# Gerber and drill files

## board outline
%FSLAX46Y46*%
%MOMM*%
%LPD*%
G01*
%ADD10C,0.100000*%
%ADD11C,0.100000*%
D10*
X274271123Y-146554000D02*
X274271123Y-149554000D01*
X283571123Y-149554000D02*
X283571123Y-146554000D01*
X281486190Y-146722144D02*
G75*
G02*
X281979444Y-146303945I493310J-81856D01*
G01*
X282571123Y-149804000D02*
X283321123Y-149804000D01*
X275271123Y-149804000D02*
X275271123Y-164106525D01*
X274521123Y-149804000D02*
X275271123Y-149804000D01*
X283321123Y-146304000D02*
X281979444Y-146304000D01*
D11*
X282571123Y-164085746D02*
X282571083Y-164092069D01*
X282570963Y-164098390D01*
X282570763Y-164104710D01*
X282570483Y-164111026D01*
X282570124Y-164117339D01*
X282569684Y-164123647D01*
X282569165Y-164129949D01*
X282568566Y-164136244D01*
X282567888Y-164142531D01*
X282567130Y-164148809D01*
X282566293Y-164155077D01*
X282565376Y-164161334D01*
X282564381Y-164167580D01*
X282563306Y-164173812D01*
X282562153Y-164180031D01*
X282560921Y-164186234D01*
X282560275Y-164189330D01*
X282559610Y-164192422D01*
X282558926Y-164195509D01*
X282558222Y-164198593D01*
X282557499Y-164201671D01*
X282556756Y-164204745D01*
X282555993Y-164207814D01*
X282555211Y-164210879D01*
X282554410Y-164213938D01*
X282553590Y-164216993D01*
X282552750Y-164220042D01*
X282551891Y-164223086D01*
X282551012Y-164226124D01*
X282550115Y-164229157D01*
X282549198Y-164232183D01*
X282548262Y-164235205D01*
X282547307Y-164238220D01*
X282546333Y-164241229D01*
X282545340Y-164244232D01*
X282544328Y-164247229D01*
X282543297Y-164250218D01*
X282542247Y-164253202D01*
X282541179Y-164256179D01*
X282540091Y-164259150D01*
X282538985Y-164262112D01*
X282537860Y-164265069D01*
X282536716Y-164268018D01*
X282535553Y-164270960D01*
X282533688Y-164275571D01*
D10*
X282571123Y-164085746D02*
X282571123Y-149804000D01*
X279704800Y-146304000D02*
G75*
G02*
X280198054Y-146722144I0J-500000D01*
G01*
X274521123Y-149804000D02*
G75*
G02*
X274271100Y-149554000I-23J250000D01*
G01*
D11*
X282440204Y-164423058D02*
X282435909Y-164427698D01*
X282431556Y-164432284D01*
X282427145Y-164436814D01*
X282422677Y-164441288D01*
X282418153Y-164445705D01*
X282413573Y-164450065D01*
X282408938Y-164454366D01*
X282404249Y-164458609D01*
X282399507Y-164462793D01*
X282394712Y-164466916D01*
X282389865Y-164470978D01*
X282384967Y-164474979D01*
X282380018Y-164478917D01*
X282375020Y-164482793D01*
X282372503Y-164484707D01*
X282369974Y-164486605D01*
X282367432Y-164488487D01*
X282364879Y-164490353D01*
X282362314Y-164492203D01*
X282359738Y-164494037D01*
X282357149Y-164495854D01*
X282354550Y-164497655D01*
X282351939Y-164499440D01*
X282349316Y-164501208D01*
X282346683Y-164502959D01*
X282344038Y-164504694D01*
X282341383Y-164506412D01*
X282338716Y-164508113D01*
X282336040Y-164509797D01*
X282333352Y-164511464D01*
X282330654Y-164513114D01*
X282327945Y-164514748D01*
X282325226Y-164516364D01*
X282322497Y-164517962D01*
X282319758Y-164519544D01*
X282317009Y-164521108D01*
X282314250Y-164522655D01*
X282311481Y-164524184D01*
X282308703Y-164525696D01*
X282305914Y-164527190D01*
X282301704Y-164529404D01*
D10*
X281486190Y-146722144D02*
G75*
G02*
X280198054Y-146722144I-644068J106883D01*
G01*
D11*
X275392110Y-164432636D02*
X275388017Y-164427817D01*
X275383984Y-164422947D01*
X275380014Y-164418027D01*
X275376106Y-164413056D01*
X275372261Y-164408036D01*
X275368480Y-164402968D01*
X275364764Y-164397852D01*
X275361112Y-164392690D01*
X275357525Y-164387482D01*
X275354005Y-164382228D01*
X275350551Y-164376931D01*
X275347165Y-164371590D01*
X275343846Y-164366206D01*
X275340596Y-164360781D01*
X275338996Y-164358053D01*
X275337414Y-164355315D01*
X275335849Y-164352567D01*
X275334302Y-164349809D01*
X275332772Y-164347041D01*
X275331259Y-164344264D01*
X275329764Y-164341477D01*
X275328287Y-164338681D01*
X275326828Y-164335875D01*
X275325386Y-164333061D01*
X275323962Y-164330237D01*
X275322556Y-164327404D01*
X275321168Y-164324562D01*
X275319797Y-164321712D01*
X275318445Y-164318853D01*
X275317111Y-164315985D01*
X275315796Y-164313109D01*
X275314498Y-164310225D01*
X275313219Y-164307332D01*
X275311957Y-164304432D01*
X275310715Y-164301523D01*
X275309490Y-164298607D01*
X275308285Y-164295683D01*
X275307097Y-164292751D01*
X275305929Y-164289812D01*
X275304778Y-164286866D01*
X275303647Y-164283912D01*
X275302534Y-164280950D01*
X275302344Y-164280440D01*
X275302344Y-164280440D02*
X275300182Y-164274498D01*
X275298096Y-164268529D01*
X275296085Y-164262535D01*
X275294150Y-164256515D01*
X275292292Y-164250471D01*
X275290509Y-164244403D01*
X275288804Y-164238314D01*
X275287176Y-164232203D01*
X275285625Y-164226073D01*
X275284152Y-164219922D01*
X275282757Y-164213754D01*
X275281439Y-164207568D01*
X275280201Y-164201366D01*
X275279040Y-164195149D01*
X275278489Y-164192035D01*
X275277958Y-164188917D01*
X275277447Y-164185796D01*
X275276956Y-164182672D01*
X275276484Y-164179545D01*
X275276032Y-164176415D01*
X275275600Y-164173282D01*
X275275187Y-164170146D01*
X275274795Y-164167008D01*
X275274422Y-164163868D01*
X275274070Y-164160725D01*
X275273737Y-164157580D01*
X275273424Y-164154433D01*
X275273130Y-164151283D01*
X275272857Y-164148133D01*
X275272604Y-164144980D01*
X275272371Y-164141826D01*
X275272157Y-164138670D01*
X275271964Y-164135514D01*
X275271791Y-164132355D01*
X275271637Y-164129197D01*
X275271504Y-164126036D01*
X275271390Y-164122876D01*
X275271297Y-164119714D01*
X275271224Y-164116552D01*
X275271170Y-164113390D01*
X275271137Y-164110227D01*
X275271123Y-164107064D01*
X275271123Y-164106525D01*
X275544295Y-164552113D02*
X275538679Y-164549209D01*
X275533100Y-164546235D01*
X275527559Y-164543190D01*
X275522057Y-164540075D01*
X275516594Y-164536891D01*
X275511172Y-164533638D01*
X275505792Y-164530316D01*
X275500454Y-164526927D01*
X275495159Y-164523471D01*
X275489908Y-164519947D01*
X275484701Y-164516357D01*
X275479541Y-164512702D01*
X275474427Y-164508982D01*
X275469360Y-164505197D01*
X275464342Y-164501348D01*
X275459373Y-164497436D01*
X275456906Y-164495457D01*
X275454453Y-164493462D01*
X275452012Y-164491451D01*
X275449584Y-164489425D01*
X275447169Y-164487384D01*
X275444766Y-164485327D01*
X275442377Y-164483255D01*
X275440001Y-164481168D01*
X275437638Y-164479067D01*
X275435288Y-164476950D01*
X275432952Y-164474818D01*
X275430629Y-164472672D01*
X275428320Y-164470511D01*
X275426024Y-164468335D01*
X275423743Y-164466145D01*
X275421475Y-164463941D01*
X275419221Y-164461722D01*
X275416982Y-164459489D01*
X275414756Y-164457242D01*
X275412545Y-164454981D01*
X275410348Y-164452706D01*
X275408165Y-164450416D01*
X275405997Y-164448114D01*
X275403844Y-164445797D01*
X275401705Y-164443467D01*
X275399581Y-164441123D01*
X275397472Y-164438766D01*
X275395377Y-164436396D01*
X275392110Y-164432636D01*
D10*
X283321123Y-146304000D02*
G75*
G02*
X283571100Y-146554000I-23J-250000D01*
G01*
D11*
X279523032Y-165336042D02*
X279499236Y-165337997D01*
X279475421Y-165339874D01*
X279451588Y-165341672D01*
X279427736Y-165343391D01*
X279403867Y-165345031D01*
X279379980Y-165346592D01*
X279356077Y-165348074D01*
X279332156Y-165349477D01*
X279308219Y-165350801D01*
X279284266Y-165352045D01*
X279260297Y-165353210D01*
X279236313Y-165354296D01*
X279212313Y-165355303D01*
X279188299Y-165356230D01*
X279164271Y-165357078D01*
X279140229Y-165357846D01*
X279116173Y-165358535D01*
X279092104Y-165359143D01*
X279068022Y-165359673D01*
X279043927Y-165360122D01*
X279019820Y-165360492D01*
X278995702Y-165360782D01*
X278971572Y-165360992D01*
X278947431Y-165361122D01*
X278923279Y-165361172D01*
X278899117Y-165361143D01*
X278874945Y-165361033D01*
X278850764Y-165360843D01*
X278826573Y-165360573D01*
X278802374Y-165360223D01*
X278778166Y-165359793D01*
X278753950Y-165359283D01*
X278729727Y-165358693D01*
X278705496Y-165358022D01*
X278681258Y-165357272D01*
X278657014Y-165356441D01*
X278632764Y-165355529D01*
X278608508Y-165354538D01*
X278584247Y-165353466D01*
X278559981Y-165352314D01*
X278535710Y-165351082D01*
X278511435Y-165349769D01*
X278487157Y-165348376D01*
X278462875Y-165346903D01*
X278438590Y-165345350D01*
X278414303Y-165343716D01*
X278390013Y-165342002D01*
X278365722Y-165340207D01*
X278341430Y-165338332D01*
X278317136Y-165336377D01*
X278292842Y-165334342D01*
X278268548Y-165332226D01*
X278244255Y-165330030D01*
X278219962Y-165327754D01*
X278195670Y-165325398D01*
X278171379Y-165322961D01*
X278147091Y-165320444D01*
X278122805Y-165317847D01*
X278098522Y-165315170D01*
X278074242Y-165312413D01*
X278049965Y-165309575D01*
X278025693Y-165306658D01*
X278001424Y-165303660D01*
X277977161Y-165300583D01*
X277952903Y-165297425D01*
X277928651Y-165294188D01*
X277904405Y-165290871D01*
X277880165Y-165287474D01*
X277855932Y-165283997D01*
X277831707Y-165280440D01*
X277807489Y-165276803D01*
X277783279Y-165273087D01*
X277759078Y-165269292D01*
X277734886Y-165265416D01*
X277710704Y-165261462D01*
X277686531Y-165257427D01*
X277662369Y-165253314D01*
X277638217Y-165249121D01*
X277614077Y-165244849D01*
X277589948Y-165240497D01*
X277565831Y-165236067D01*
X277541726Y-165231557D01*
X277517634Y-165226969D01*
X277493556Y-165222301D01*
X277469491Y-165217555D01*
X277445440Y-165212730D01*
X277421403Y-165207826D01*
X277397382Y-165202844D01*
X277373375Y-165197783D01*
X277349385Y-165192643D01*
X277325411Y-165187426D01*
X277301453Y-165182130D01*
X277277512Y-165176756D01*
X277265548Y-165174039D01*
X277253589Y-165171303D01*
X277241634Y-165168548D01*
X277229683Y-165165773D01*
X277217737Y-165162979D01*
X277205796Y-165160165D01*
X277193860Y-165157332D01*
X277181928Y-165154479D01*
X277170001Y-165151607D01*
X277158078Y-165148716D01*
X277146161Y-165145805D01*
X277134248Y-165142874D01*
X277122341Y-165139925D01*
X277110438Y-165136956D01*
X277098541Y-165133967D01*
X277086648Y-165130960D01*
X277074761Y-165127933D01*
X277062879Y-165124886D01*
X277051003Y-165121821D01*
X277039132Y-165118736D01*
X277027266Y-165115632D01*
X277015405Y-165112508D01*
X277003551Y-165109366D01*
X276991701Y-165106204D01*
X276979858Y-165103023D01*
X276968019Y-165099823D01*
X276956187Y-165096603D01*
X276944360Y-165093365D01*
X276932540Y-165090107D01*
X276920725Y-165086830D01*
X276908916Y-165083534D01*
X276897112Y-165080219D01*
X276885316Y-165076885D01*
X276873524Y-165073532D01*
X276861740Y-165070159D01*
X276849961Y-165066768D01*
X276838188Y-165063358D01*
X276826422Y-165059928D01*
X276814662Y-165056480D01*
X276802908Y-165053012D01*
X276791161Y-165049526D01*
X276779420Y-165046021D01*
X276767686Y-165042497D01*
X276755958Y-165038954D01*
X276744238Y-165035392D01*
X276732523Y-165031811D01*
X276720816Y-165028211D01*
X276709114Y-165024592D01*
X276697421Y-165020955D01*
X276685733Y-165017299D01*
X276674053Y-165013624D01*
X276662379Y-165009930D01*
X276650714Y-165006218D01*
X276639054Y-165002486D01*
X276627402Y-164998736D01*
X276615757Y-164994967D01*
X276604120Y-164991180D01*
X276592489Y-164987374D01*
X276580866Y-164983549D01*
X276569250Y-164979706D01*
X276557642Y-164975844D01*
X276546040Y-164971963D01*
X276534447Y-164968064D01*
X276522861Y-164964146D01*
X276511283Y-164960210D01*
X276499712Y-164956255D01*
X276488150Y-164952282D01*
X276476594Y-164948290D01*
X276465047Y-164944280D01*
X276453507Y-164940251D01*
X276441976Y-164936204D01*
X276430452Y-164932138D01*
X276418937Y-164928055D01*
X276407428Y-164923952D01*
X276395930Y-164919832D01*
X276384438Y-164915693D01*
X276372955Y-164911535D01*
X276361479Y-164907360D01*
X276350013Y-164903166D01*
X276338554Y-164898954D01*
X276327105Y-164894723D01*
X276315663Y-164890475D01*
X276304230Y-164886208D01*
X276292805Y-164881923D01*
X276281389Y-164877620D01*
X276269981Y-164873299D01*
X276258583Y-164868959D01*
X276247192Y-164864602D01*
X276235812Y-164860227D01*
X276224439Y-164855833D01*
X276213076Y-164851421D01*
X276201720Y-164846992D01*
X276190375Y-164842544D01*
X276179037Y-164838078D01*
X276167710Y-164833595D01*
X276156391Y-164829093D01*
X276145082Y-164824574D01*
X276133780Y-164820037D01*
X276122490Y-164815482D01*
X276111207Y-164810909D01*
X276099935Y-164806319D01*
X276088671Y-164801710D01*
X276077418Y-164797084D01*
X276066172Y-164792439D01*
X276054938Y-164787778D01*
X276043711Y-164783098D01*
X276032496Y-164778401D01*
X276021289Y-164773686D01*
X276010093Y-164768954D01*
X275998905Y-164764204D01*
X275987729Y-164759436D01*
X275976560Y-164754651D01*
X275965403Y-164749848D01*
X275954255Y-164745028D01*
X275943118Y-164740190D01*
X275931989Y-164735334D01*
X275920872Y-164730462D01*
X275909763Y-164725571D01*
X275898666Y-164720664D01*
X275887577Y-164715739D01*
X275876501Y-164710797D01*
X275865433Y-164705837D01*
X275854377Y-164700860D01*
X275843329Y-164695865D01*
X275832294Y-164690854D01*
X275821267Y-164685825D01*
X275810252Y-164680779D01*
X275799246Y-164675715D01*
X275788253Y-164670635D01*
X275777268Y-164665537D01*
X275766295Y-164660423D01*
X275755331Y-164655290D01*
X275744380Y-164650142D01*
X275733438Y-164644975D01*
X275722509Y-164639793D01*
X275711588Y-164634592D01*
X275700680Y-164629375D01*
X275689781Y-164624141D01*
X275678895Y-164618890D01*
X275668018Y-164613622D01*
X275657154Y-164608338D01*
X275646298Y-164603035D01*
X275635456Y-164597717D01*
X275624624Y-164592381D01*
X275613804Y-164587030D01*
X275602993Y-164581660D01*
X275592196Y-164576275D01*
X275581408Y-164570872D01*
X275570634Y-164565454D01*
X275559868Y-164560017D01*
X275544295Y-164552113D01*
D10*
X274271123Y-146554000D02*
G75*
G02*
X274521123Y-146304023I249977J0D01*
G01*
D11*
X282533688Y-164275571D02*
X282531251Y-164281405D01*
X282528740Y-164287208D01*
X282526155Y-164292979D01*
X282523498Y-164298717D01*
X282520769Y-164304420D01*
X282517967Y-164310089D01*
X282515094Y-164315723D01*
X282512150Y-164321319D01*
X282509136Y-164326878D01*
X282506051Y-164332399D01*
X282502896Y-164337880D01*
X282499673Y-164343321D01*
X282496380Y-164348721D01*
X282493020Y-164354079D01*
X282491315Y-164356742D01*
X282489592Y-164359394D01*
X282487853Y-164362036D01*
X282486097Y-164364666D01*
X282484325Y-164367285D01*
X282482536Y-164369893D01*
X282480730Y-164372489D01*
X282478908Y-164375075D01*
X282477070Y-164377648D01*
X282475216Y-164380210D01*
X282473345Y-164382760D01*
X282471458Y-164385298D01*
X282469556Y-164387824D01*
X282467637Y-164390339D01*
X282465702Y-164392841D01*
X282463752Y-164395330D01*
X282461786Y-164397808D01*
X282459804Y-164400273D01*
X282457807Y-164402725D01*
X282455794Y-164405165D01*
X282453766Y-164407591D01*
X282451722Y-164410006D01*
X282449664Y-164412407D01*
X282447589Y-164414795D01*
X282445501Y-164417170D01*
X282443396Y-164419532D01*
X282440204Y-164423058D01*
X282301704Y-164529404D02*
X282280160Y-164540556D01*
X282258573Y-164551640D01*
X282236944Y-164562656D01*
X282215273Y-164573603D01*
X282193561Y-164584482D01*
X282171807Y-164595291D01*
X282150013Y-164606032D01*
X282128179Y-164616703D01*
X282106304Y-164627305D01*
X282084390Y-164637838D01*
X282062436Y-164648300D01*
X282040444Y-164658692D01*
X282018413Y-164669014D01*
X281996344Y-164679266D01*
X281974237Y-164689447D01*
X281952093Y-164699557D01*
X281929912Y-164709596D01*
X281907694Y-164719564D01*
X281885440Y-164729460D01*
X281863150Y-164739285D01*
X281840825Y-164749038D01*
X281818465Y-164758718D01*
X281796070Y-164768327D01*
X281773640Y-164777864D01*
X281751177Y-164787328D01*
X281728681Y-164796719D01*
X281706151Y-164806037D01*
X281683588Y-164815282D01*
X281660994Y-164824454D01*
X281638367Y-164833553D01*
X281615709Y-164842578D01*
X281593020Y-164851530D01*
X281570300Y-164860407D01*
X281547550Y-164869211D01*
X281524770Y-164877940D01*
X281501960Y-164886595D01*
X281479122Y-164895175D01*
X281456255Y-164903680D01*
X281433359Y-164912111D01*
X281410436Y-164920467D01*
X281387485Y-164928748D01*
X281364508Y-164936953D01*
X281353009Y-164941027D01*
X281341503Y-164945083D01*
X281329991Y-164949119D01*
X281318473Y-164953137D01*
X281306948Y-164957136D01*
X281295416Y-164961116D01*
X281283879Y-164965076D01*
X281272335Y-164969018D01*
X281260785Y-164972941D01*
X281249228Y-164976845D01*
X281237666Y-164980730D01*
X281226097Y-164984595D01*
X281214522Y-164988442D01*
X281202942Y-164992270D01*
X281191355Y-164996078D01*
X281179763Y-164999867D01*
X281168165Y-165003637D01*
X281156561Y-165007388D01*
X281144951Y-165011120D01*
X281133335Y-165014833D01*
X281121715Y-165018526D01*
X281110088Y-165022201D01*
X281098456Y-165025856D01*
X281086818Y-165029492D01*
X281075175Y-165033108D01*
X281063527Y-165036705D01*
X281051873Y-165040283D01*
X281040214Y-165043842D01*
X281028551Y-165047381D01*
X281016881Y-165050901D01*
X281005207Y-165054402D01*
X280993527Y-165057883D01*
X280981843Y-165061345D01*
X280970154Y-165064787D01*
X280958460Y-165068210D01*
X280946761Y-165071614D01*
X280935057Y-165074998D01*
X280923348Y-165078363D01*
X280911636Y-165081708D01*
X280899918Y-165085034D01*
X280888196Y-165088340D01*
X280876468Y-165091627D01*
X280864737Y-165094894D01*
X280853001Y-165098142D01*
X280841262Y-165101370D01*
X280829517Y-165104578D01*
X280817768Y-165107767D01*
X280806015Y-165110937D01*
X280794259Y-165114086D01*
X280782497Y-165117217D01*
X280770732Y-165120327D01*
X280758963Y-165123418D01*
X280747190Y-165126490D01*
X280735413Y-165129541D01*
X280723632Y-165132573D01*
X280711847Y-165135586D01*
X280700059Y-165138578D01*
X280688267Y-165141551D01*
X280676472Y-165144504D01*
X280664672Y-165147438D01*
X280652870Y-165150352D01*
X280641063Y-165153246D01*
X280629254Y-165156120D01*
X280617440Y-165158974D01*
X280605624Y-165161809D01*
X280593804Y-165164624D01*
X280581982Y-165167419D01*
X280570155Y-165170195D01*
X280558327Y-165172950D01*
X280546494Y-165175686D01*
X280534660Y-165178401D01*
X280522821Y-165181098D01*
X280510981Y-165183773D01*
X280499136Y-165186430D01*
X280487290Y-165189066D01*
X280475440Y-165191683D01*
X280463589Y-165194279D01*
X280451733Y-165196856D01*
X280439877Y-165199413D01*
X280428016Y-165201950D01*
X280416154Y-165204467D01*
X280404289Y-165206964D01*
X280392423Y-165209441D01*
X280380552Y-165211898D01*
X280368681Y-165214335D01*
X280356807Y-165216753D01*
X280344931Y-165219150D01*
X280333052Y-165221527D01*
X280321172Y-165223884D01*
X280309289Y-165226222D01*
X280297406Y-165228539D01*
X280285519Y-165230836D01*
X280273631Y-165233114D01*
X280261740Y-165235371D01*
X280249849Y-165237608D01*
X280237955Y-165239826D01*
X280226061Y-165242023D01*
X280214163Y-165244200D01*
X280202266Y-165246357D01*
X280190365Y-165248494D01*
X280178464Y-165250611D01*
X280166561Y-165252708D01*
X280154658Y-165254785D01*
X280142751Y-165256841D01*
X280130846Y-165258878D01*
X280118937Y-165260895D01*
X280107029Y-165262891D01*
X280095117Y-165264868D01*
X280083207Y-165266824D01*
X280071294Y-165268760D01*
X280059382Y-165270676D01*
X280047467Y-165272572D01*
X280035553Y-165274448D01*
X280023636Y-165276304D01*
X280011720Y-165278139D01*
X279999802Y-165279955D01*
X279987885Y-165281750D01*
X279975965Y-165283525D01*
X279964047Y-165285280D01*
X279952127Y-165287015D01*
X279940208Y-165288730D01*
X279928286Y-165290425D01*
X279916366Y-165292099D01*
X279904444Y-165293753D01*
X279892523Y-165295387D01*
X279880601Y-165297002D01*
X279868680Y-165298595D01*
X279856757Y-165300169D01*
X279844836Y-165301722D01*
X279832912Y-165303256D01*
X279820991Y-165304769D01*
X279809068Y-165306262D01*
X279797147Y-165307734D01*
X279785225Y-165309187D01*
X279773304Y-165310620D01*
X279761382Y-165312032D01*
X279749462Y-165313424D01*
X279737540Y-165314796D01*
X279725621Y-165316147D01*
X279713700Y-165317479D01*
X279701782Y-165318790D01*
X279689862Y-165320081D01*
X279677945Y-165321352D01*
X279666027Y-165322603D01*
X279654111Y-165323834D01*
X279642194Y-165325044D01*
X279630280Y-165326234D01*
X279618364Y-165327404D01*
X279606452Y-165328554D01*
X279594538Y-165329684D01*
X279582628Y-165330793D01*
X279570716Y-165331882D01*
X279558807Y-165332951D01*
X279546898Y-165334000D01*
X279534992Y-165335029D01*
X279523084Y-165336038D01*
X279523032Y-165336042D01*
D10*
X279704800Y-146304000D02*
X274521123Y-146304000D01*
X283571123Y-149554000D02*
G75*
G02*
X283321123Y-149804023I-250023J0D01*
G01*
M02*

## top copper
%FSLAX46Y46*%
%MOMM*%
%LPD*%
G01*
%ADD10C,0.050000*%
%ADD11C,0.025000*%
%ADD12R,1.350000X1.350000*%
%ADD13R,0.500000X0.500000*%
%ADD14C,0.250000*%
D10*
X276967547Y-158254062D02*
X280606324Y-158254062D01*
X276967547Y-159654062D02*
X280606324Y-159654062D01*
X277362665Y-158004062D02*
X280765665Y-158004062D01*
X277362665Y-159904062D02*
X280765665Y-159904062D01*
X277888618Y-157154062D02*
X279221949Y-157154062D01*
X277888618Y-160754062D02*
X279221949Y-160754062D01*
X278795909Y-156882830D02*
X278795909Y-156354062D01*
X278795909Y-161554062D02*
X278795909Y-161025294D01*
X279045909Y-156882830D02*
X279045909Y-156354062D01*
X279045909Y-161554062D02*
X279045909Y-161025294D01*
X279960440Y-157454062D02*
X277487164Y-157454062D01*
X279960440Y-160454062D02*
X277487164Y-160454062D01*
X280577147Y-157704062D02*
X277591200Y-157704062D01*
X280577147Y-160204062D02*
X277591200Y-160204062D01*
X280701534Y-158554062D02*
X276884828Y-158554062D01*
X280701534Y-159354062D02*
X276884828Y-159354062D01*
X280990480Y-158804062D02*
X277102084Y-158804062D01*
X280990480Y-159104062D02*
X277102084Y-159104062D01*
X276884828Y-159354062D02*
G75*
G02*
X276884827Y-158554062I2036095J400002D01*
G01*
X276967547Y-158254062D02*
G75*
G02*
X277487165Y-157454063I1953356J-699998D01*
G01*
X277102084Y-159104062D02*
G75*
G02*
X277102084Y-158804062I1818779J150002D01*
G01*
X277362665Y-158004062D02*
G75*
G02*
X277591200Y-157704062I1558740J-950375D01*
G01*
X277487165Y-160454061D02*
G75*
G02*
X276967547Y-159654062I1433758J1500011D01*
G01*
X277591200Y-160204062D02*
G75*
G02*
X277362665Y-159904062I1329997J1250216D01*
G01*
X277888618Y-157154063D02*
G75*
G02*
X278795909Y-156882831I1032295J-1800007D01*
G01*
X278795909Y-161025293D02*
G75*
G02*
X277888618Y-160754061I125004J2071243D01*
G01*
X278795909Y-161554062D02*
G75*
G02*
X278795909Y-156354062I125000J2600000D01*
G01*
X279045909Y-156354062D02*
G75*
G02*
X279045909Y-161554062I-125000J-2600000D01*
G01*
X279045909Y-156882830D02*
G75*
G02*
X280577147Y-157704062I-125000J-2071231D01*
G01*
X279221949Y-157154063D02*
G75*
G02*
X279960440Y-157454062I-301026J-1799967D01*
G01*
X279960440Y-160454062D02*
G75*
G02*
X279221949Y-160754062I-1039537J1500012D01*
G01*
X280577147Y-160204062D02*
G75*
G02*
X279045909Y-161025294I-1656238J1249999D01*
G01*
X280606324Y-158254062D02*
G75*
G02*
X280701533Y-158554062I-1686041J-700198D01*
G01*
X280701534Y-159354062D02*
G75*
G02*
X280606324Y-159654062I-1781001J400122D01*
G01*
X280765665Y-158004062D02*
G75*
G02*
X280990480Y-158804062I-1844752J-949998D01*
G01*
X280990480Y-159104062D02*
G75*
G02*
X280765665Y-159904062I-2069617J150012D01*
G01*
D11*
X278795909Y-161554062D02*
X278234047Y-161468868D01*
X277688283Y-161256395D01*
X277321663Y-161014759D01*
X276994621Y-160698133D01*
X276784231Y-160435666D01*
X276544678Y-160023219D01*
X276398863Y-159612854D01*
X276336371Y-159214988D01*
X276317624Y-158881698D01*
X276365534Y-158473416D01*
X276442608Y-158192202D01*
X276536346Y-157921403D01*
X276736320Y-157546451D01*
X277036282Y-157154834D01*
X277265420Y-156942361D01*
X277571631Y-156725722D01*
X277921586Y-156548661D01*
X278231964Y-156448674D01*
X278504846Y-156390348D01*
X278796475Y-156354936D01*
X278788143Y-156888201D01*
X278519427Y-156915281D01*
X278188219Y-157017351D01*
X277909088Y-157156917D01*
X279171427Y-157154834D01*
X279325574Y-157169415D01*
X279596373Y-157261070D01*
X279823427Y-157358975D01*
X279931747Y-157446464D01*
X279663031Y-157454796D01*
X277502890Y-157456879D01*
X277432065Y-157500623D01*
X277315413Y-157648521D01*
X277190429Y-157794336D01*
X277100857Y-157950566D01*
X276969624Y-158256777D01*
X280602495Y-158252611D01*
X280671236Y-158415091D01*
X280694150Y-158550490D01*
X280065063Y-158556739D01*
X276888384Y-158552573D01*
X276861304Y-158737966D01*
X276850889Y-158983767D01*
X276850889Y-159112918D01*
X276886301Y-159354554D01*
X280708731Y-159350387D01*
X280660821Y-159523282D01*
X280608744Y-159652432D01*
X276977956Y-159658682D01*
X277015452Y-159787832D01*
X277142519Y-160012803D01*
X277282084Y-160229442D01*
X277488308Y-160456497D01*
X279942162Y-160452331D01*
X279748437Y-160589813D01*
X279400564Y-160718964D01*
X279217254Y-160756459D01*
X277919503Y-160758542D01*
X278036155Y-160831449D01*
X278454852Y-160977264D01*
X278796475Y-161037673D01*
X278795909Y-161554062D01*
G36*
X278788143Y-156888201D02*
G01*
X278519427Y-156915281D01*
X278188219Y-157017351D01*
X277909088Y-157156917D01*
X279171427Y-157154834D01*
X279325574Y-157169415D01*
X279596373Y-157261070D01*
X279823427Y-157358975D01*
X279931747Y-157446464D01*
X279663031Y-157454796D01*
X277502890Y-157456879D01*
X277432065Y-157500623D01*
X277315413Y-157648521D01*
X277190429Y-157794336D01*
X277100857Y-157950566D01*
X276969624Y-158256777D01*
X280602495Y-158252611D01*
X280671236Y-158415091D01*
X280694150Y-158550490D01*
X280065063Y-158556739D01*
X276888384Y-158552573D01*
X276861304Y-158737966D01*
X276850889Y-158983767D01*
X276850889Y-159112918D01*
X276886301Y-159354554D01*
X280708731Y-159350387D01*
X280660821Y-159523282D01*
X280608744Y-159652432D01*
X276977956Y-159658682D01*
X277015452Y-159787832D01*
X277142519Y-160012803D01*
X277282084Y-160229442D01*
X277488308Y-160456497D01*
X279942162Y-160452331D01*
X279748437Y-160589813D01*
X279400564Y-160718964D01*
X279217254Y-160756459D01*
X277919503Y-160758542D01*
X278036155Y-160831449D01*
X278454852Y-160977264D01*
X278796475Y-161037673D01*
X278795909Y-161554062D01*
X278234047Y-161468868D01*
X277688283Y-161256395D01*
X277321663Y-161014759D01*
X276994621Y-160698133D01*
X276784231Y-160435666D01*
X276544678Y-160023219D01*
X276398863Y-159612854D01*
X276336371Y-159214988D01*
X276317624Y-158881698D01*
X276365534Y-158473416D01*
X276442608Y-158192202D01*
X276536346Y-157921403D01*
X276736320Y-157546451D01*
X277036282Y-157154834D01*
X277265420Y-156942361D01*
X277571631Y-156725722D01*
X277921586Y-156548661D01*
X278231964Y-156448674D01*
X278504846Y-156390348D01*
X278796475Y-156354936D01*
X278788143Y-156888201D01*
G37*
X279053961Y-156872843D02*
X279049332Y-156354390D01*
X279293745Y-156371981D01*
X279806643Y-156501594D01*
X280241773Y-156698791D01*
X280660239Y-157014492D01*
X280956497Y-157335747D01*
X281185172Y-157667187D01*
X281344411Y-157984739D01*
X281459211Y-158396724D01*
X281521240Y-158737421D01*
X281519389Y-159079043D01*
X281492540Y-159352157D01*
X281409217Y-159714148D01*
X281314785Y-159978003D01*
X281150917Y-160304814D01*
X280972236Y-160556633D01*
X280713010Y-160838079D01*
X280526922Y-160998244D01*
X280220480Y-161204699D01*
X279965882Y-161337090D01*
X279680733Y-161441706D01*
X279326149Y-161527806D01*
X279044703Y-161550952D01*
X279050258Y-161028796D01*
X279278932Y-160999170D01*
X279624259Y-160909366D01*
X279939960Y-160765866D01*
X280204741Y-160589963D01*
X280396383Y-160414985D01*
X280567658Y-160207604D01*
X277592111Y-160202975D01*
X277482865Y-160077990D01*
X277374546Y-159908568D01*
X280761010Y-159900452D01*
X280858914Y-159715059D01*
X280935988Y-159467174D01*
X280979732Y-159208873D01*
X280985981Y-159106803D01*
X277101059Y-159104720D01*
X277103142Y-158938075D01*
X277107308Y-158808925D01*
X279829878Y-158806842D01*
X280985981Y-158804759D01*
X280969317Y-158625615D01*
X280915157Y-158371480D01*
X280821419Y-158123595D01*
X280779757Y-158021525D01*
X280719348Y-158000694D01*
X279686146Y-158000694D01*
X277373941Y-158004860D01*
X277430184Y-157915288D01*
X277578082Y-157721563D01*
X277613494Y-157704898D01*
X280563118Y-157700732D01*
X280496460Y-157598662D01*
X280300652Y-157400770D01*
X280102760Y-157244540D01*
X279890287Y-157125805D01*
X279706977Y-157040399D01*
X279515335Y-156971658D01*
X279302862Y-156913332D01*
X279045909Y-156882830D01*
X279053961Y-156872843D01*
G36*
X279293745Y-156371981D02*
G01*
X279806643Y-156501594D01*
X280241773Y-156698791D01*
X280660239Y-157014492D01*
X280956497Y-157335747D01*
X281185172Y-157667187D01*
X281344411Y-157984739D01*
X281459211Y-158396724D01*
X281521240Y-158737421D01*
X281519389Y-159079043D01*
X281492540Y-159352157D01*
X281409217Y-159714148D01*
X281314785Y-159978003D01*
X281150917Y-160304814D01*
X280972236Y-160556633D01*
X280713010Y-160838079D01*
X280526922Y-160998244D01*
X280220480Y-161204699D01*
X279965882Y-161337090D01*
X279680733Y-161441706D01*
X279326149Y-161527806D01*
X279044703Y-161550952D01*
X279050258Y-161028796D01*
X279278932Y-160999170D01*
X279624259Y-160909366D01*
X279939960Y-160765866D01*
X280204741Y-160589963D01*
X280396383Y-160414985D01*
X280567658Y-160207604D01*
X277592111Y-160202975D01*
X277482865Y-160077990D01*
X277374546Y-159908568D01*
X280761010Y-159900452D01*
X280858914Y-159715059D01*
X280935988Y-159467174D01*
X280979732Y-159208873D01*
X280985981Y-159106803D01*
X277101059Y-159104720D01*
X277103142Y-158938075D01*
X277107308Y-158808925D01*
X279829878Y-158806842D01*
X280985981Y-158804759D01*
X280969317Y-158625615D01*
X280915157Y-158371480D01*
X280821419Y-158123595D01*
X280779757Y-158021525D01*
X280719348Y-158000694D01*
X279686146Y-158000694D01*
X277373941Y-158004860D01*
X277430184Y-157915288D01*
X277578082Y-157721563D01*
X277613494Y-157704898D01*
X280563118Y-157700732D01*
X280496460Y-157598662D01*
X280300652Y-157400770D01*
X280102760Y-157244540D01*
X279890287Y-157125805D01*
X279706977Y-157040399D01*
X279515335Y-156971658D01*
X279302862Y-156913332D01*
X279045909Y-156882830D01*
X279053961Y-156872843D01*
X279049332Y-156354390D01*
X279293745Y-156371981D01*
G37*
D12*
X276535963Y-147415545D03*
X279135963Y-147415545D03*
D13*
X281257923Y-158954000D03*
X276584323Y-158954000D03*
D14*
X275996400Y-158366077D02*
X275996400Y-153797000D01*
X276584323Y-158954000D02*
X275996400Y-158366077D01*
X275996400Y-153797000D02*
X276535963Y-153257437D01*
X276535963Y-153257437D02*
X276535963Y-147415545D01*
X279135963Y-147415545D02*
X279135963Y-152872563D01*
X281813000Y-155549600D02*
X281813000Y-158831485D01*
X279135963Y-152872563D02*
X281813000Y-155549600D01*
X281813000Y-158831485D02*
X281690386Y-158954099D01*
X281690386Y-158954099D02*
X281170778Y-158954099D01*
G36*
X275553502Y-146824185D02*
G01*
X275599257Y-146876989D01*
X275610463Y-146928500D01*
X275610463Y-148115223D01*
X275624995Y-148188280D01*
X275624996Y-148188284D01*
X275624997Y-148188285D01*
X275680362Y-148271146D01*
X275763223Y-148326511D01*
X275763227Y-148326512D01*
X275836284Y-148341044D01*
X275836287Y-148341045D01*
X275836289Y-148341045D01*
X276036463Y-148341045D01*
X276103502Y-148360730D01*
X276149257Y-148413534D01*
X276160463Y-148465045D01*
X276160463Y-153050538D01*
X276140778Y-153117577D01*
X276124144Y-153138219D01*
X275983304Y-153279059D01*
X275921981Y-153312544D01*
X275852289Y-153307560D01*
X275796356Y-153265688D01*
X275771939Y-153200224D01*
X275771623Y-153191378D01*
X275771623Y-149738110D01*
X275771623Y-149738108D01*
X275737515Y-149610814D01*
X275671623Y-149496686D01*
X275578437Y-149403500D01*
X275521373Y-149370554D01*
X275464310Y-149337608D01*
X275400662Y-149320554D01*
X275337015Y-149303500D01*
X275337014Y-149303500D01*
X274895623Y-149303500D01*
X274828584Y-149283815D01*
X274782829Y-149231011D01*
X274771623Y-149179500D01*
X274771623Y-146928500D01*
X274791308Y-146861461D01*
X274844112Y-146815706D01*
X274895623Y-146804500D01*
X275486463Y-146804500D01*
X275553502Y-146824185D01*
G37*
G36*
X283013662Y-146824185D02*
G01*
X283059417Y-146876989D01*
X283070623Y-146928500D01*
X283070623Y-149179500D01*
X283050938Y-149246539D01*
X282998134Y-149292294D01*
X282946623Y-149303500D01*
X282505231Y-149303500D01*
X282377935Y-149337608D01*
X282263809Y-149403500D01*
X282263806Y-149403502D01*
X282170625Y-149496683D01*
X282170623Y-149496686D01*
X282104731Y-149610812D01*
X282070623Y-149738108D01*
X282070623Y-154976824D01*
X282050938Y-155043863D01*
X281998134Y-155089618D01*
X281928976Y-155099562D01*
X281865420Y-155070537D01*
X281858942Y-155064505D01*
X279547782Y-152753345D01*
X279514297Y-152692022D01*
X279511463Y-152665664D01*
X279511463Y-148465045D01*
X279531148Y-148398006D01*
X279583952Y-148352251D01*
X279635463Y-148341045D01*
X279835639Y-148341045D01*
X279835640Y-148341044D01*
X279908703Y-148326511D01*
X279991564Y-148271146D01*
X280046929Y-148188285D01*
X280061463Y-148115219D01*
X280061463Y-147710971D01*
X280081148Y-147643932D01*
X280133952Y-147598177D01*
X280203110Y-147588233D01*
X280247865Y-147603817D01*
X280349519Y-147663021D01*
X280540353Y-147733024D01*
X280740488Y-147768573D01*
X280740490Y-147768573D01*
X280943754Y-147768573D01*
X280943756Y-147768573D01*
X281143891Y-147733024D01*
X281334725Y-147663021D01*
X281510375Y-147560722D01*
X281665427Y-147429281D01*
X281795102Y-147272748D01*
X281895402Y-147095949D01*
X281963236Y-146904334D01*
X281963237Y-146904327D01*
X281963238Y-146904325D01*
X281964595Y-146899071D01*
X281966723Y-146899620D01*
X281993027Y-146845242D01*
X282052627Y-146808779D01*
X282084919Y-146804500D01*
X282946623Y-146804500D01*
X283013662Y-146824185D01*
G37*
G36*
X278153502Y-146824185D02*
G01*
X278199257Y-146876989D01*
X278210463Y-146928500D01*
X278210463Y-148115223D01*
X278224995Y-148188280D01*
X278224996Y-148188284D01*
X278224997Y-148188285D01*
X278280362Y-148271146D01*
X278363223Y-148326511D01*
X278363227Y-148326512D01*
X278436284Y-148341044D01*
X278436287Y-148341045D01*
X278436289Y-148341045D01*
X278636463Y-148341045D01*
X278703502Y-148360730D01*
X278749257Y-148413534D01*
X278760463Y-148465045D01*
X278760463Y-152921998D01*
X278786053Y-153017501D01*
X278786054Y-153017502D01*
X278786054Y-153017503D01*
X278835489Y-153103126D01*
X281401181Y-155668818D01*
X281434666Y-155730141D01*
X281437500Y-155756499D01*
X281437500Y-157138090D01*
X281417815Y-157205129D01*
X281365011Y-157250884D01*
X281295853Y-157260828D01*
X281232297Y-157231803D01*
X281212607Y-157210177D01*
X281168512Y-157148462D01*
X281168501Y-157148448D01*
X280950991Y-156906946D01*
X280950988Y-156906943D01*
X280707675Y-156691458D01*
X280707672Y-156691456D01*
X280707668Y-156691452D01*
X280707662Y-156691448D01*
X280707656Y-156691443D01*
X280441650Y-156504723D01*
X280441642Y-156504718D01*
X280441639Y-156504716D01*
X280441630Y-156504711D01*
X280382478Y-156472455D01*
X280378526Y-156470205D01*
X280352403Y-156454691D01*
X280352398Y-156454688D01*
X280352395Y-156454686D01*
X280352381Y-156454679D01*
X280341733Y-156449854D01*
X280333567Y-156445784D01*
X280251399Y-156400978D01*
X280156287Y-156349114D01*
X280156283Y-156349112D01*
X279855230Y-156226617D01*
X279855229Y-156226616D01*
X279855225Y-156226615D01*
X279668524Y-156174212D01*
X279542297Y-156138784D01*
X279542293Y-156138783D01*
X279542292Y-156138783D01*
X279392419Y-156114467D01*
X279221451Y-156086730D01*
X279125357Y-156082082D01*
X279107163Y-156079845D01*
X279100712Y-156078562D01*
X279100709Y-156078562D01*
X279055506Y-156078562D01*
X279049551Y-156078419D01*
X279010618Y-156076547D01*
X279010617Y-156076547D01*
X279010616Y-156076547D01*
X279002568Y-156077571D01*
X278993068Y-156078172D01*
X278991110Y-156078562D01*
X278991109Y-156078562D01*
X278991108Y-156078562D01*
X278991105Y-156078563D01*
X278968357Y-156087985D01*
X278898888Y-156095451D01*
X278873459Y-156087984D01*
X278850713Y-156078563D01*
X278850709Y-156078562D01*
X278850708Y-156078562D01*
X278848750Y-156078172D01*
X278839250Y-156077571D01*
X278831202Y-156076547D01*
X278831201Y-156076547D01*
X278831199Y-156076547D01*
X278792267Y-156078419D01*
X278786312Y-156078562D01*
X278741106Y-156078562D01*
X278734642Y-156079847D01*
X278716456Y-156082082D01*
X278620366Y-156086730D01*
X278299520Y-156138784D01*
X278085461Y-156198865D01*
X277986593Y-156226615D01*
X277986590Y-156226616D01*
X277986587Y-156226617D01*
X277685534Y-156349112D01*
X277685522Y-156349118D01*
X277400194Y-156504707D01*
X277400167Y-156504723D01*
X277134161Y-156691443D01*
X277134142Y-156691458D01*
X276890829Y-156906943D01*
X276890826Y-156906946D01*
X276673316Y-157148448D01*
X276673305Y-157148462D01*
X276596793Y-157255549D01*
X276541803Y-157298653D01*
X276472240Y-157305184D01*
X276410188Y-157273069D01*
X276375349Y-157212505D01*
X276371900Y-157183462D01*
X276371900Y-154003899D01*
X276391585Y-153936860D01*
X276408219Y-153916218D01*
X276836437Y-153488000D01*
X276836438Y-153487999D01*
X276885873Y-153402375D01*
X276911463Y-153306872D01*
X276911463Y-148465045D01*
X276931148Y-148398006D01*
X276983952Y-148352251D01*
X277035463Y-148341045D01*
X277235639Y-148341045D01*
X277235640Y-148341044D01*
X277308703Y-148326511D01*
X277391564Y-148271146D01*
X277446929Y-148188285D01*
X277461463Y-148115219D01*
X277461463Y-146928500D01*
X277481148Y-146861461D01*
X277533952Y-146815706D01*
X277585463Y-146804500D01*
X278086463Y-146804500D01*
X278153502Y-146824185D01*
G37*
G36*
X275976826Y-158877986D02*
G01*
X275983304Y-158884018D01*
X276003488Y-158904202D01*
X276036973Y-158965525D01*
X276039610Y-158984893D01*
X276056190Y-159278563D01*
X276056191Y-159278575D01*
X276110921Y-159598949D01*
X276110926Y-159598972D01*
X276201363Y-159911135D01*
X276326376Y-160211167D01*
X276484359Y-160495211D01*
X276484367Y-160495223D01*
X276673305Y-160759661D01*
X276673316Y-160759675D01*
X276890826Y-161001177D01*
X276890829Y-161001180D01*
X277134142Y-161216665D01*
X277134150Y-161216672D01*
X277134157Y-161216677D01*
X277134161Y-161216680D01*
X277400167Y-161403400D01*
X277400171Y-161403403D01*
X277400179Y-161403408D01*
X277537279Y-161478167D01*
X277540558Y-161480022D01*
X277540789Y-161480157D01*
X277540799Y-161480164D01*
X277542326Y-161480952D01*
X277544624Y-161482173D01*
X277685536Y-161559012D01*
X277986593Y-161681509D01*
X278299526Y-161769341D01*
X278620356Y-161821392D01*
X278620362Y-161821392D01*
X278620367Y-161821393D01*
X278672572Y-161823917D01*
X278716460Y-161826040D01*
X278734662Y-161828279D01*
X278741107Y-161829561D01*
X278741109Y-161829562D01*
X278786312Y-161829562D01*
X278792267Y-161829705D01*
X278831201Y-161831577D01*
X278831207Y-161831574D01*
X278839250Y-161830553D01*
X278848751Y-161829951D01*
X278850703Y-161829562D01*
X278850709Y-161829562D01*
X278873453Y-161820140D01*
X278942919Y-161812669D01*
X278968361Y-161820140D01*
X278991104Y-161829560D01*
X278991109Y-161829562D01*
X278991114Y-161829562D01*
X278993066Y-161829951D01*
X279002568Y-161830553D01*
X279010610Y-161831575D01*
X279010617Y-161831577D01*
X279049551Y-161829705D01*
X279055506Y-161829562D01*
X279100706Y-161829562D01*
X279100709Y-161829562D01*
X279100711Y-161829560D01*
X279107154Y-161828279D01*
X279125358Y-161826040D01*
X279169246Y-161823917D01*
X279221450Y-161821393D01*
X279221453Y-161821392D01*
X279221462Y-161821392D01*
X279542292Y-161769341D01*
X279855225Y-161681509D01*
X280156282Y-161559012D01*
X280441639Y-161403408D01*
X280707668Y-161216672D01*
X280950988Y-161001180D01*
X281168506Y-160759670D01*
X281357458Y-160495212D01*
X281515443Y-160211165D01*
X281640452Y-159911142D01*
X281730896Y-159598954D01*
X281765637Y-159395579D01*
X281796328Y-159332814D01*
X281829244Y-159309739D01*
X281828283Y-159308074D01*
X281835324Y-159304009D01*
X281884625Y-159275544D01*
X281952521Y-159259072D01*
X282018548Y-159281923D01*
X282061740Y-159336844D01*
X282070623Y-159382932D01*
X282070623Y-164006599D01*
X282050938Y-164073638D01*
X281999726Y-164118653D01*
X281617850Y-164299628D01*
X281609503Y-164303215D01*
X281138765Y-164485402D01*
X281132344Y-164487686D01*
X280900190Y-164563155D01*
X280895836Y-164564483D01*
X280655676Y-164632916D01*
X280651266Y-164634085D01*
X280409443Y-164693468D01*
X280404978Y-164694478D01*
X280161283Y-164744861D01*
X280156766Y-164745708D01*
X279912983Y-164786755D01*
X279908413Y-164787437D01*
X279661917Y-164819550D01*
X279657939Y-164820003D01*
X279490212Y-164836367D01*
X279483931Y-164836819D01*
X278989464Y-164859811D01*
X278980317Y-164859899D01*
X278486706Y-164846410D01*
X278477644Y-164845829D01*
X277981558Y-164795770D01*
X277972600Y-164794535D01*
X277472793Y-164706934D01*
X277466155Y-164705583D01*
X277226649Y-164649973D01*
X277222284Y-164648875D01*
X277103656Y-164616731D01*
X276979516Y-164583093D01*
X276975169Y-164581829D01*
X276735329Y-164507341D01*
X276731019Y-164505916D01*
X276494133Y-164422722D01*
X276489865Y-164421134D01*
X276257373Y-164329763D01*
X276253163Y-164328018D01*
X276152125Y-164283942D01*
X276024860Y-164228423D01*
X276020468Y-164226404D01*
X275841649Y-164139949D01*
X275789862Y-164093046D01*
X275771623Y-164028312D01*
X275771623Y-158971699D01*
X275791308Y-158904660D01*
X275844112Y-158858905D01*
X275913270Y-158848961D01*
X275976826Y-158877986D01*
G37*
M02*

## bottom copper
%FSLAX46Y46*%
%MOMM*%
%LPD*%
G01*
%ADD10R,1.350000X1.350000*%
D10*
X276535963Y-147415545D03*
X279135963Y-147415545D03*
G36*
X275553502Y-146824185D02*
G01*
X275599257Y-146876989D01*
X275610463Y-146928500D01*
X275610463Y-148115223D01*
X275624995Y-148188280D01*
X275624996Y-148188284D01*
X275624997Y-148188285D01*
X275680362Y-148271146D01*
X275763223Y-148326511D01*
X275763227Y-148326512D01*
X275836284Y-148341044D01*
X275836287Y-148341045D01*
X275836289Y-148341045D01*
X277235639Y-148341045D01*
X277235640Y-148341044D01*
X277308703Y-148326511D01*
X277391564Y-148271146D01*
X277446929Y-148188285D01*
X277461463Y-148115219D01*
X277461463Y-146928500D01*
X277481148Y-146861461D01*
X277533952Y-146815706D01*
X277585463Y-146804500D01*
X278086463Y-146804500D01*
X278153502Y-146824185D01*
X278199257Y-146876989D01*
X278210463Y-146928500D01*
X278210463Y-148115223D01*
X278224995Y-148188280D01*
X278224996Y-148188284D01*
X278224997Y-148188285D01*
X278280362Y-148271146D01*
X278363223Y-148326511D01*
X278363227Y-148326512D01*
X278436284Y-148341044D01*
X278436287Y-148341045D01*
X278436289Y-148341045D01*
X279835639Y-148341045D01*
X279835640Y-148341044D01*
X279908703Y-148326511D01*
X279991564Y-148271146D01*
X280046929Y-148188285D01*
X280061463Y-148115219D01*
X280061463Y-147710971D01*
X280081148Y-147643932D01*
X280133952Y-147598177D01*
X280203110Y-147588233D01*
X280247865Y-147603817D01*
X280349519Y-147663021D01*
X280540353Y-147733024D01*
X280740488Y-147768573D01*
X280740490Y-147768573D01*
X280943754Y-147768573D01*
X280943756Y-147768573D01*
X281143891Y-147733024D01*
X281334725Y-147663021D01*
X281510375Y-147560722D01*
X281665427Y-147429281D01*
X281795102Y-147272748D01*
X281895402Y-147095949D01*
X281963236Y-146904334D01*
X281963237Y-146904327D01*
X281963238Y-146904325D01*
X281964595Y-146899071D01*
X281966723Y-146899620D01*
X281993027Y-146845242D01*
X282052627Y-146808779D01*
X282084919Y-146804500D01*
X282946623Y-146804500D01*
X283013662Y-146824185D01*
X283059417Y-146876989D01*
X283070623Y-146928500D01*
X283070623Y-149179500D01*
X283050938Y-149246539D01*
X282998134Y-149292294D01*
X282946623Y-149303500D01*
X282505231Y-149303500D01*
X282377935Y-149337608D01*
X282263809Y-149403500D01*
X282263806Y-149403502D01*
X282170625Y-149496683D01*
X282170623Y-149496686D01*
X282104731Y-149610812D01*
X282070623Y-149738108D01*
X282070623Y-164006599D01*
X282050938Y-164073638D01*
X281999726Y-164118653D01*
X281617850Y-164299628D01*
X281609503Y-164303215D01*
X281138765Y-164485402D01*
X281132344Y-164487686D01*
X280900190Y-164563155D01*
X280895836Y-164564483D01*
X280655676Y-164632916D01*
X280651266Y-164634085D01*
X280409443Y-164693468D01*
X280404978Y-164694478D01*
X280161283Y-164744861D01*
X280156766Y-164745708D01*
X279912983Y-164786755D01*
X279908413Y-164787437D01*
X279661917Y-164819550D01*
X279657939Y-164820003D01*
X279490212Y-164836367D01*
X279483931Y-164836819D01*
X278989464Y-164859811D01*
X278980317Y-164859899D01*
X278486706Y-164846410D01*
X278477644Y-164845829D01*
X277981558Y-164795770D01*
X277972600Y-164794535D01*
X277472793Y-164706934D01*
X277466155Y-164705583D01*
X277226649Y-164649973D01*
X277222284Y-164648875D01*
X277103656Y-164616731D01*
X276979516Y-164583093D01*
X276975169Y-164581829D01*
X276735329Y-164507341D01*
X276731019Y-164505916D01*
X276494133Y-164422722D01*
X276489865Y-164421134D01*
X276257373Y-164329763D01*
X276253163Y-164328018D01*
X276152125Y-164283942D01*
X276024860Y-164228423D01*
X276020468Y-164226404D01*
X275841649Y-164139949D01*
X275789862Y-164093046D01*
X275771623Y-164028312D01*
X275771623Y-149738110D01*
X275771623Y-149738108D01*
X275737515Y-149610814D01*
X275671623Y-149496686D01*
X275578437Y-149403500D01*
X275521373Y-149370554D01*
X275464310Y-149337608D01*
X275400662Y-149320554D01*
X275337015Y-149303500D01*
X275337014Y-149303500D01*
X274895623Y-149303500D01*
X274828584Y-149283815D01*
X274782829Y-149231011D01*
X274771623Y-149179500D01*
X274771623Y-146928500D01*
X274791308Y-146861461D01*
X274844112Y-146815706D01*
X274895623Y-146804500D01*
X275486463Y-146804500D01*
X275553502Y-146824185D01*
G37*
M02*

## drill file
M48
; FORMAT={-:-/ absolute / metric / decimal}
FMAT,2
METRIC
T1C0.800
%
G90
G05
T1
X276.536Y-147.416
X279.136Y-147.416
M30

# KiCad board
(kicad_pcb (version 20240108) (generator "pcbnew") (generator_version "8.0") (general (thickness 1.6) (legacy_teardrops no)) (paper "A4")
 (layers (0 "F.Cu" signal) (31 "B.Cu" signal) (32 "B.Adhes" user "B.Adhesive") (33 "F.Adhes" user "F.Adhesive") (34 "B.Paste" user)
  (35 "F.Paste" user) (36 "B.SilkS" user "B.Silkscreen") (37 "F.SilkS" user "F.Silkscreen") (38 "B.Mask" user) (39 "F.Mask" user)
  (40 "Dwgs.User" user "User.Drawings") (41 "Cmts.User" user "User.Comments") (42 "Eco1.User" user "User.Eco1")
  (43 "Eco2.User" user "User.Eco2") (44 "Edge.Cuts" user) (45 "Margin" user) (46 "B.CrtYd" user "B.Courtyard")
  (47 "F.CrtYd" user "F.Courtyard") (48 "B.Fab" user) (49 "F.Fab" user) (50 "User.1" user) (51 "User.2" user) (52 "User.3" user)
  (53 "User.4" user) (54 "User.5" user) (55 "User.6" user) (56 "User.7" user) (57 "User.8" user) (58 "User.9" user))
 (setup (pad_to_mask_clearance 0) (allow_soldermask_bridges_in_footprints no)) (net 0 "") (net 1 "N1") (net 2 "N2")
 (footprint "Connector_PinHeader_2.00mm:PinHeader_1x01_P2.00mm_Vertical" (layer "F.Cu") (at 276.535963 147.415545)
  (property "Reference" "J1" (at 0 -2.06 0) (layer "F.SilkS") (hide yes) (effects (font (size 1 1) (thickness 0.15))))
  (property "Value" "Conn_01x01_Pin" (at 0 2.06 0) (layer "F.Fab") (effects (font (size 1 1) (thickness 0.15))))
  (pad "1" thru_hole rect (at 0 0) (size 1.35 1.35) (drill 0.8) (layers "*.Cu" "*.Mask") (remove_unused_layers no) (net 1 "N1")))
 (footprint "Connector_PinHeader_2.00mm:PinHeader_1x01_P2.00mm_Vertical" (layer "F.Cu") (at 279.135963 147.415545)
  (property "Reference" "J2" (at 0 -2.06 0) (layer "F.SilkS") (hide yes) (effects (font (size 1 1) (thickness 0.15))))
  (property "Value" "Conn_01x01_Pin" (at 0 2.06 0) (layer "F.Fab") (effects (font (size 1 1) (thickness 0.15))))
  (pad "1" thru_hole rect (at 0 0) (size 1.35 1.35) (drill 0.8) (layers "*.Cu" "*.Mask") (remove_unused_layers no) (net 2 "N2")))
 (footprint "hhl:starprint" (layer "F.Cu") (at 278.921123 158.954 180)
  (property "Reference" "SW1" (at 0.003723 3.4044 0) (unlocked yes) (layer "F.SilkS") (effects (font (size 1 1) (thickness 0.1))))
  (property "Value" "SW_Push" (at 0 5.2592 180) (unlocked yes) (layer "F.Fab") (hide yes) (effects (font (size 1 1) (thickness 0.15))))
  (fp_line (start 1.953576 0.699938) (end -1.685201 0.699938) (stroke (width 0.05) (type solid)) (layer "F.Cu"))
  (fp_line (start 1.953576 -0.700062) (end -1.685201 -0.700062) (stroke (width 0.05) (type solid)) (layer "F.Cu"))
  (fp_line (start 1.558458 0.949938) (end -1.844542 0.949938) (stroke (width 0.05) (type solid)) (layer "F.Cu"))
  (fp_line (start 1.558458 -0.950062) (end -1.844542 -0.950062) (stroke (width 0.05) (type solid)) (layer "F.Cu"))
  (fp_line (start 1.032505 1.799938) (end -0.300826 1.799938) (stroke (width 0.05) (type solid)) (layer "F.Cu"))
  (fp_line (start 1.032505 -1.800062) (end -0.300826 -1.800062) (stroke (width 0.05) (type solid)) (layer "F.Cu"))
  (fp_line (start 0.125214 2.07117) (end 0.125214 2.599938) (stroke (width 0.05) (type solid)) (layer "F.Cu"))
  (fp_line (start 0.125214 -2.600062) (end 0.125214 -2.071294) (stroke (width 0.05) (type solid)) (layer "F.Cu"))
  (fp_line (start -0.124786 2.07117) (end -0.124786 2.599938) (stroke (width 0.05) (type solid)) (layer "F.Cu"))
  (fp_line (start -0.124786 -2.600062) (end -0.124786 -2.071294) (stroke (width 0.05) (type solid)) (layer "F.Cu"))
  (fp_line (start -1.039317 1.499938) (end 1.433959 1.499938) (stroke (width 0.05) (type solid)) (layer "F.Cu"))
  (fp_line (start -1.039317 -1.500062) (end 1.433959 -1.500062) (stroke (width 0.05) (type solid)) (layer "F.Cu"))
  (fp_line (start -1.656024 1.249938) (end 1.329923 1.249938) (stroke (width 0.05) (type solid)) (layer "F.Cu"))
  (fp_line (start -1.656024 -1.250062) (end 1.329923 -1.250062) (stroke (width 0.05) (type solid)) (layer "F.Cu"))
  (fp_line (start -1.780411 0.399938) (end 2.036295 0.399938) (stroke (width 0.05) (type solid)) (layer "F.Cu"))
  (fp_line (start -1.780411 -0.400062) (end 2.036295 -0.400062) (stroke (width 0.05) (type solid)) (layer "F.Cu"))
  (fp_line (start -2.069357 0.149938) (end 1.819039 0.149938) (stroke (width 0.05) (type solid)) (layer "F.Cu"))
  (fp_line (start -2.069357 -0.150062) (end 1.819039 -0.150062) (stroke (width 0.05) (type solid)) (layer "F.Cu"))
  (fp_arc (start 2.036295 -0.400062) (mid 2.075214 -0.000062) (end 2.036295 0.399938) (stroke (width 0.05) (type solid)) (layer "F.Cu"))
  (fp_arc (start 1.953576 0.699938) (mid 1.740364 1.130203) (end 1.433958 1.499937) (stroke (width 0.05) (type solid)) (layer "F.Cu"))
  (fp_arc (start 1.819039 -0.150062) (mid 1.825214 -0.000062) (end 1.819039 0.149938) (stroke (width 0.05) (type solid)) (layer "F.Cu"))
  (fp_arc (start 1.558458 0.949938) (mid 1.451958 1.105855) (end 1.329923 1.249938) (stroke (width 0.05) (type solid)) (layer "F.Cu"))
  (fp_arc (start 1.433958 -1.500061) (mid 1.740364 -1.130327) (end 1.953577 -0.700062) (stroke (width 0.05) (type solid)) (layer "F.Cu"))
  (fp_arc (start 1.329923 -1.250062) (mid 1.451959 -1.10598) (end 1.558458 -0.950062) (stroke (width 0.05) (type solid)) (layer "F.Cu"))
  (fp_arc (start 1.032505 1.799937) (mid 0.594539 1.988002) (end 0.125214 2.071169) (stroke (width 0.05) (type solid)) (layer "F.Cu"))
  (fp_arc (start 0.125214 -2.071293) (mid 0.594539 -1.988126) (end 1.032505 -1.800061) (stroke (width 0.05) (type solid)) (layer "F.Cu"))
  (fp_arc (start 0.125214 -2.600062) (mid 2.603217 -0.000062) (end 0.125214 2.599938) (stroke (width 0.05) (type solid)) (layer "F.Cu"))
  (fp_arc (start -0.124786 2.599938) (mid -2.602789 -0.000062) (end -0.124786 -2.600062) (stroke (width 0.05) (type solid)) (layer "F.Cu"))
  (fp_arc (start -0.124786 2.07117) (mid -0.980504 1.828549) (end -1.656024 1.249938) (stroke (width 0.05) (type solid)) (layer "F.Cu"))
  (fp_arc (start -0.300826 1.799937) (mid -0.68665 1.690749) (end -1.039316 1.499937) (stroke (width 0.05) (type solid)) (layer "F.Cu"))
  (fp_arc (start -1.039317 -1.500062) (mid -0.68665 -1.690873) (end -0.300826 -1.800062) (stroke (width 0.05) (type solid)) (layer "F.Cu"))
  (fp_arc (start -1.656024 -1.250062) (mid -0.980504 -1.828673) (end -0.124786 -2.071294) (stroke (width 0.05) (type solid)) (layer "F.Cu"))
  (fp_arc (start -1.685201 0.699938) (mid -1.739283 0.551994) (end -1.780411 0.399938) (stroke (width 0.05) (type solid)) (layer "F.Cu"))
  (fp_arc (start -1.780411 -0.400062) (mid -1.739284 -0.552118) (end -1.685201 -0.700062) (stroke (width 0.05) (type solid)) (layer "F.Cu"))
  (fp_arc (start -1.844542 0.949938) (mid -1.997407 0.561307) (end -2.069357 0.149938) (stroke (width 0.05) (type solid)) (layer "F.Cu"))
  (fp_arc (start -2.069357 -0.150062) (mid -1.997406 -0.561431) (end -1.844542 -0.950062) (stroke (width 0.05) (type solid)) (layer "F.Cu"))
  (fp_poly
   (pts (xy 0.125214 -2.600062) (xy 0.687076 -2.514868) (xy 1.23284 -2.302395) (xy 1.59946 -2.060759) (xy 1.926502 -1.744133)
    (xy 2.136892 -1.481666) (xy 2.376445 -1.069219) (xy 2.52226 -0.658854) (xy 2.584752 -0.260988) (xy 2.603499 0.072302)
    (xy 2.555589 0.480584) (xy 2.478515 0.761798) (xy 2.384777 1.032597) (xy 2.184803 1.407549) (xy 1.884841 1.799166)
    (xy 1.655703 2.011639) (xy 1.349492 2.228278) (xy 0.999537 2.405339) (xy 0.689159 2.505326) (xy 0.416277 2.563652)
    (xy 0.124648 2.599064) (xy 0.13298 2.065799) (xy 0.401696 2.038719) (xy 0.732904 1.936649) (xy 1.012035 1.797083)
    (xy -0.250304 1.799166) (xy -0.404451 1.784585) (xy -0.67525 1.69293) (xy -0.902304 1.595025) (xy -1.010624 1.507536)
    (xy -0.741908 1.499204) (xy 1.418233 1.497121) (xy 1.489058 1.453377) (xy 1.60571 1.305479) (xy 1.730694 1.159664)
    (xy 1.820266 1.003434) (xy 1.951499 0.697223) (xy -1.681372 0.701389) (xy -1.750113 0.538909) (xy -1.773027 0.40351)
    (xy -1.14394 0.397261) (xy 2.032739 0.401427) (xy 2.059819 0.216034) (xy 2.070234 -0.029767) (xy 2.070234 -0.158918)
    (xy 2.034822 -0.400554) (xy -1.787608 -0.396387) (xy -1.739698 -0.569282) (xy -1.687621 -0.698432) (xy 1.943167 -0.704682)
    (xy 1.905671 -0.833832) (xy 1.778604 -1.058803) (xy 1.639039 -1.275442) (xy 1.432815 -1.502497) (xy -1.021039 -1.498331)
    (xy -0.827314 -1.635813) (xy -0.479441 -1.764964) (xy -0.296131 -1.802459) (xy 1.00162 -1.804542) (xy 0.884968 -1.877449)
    (xy 0.466271 -2.023264) (xy 0.124648 -2.083673))
   (stroke (width 0.025) (type solid)) (fill solid) (layer "F.Cu"))
  (fp_poly
   (pts (xy -0.132838 2.081157) (xy -0.128209 2.59961) (xy -0.372622 2.582019) (xy -0.88552 2.452406) (xy -1.32065 2.255209)
    (xy -1.739116 1.939508) (xy -2.035374 1.618253) (xy -2.264049 1.286813) (xy -2.423288 0.969261) (xy -2.538088 0.557276)
    (xy -2.600117 0.216579) (xy -2.598266 -0.125043) (xy -2.571417 -0.398157) (xy -2.488094 -0.760148) (xy -2.393662 -1.024003)
    (xy -2.229794 -1.350814) (xy -2.051113 -1.602633) (xy -1.791887 -1.884079) (xy -1.605799 -2.044244) (xy -1.299357 -2.250699)
    (xy -1.044759 -2.38309) (xy -0.75961 -2.487706) (xy -0.405026 -2.573806) (xy -0.12358 -2.596952) (xy -0.129135 -2.074796)
    (xy -0.357809 -2.04517) (xy -0.703136 -1.955366) (xy -1.018837 -1.811866) (xy -1.283618 -1.635963) (xy -1.47526 -1.460985)
    (xy -1.646535 -1.253604) (xy 1.329012 -1.248975) (xy 1.438258 -1.12399) (xy 1.546577 -0.954568) (xy -1.839887 -0.946452)
    (xy -1.937791 -0.761059) (xy -2.014865 -0.513174) (xy -2.058609 -0.254873) (xy -2.064858 -0.152803) (xy 1.820064 -0.15072)
    (xy 1.817981 0.015925) (xy 1.813815 0.145075) (xy -0.908755 0.147158) (xy -2.064858 0.149241) (xy -2.048194 0.328385)
    (xy -1.994034 0.58252) (xy -1.900296 0.830405) (xy -1.858634 0.932475) (xy -1.798225 0.953306) (xy -0.765023 0.953306)
    (xy 1.547182 0.94914) (xy 1.490939 1.038712) (xy 1.343041 1.232437) (xy 1.307629 1.249102) (xy -1.641995 1.253268)
    (xy -1.575337 1.355338) (xy -1.379529 1.55323) (xy -1.181637 1.70946) (xy -0.969164 1.828195) (xy -0.785854 1.913601)
    (xy -0.594212 1.982342) (xy -0.381739 2.040668) (xy -0.124786 2.07117))
   (stroke (width 0.025) (type solid)) (fill solid) (layer "F.Cu"))
  (pad "1" smd rect (at -2.3368 0 180) (size 0.5 0.5) (layers "F.Cu") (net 2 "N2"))
  (pad "2" smd rect (at 2.3368 0 180) (size 0.5 0.5) (layers "F.Cu") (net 1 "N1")))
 (gr_line (start 274.271123 146.554) (end 274.271123 149.554) (stroke (width 0.1) (type solid)) (layer "Edge.Cuts"))
 (gr_line (start 283.571123 149.554) (end 283.571123 146.554) (stroke (width 0.1) (type solid)) (layer "Edge.Cuts"))
 (gr_arc (start 281.48619 146.722144) (mid 281.656126 146.422611) (end 281.979444 146.304) (stroke (width 0.1) (type solid))
  (layer "Edge.Cuts"))
 (gr_line (start 282.571123 149.804) (end 283.321123 149.804) (stroke (width 0.1) (type solid)) (layer "Edge.Cuts"))
 (gr_line (start 275.271123 149.804) (end 275.271123 164.106525) (stroke (width 0.1) (type solid)) (layer "Edge.Cuts"))
 (gr_line (start 274.521123 149.804) (end 275.271123 149.804) (stroke (width 0.1) (type solid)) (layer "Edge.Cuts"))
 (gr_line (start 283.321123 146.304) (end 281.979444 146.304) (stroke (width 0.1) (type solid)) (layer "Edge.Cuts"))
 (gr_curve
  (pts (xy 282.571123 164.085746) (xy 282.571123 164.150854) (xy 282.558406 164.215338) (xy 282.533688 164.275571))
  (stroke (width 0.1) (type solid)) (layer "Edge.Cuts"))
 (gr_line (start 282.571123 164.085746) (end 282.571123 149.804) (stroke (width 0.1) (type solid)) (layer "Edge.Cuts"))
 (gr_arc (start 279.7048 146.304) (mid 280.028133 146.422594) (end 280.198054 146.722144) (stroke (width 0.1) (type solid))
  (layer "Edge.Cuts"))
 (gr_arc (start 274.521123 149.804) (mid 274.344346 149.730777) (end 274.271123 149.554) (stroke (width 0.1) (type solid))
  (layer "Edge.Cuts"))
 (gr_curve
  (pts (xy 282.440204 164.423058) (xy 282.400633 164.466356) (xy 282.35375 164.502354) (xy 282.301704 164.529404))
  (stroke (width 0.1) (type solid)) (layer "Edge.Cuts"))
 (gr_arc (start 281.48619 146.722144) (mid 280.842122 147.268137) (end 280.198054 146.722144) (stroke (width 0.1) (type solid))
  (layer "Edge.Cuts"))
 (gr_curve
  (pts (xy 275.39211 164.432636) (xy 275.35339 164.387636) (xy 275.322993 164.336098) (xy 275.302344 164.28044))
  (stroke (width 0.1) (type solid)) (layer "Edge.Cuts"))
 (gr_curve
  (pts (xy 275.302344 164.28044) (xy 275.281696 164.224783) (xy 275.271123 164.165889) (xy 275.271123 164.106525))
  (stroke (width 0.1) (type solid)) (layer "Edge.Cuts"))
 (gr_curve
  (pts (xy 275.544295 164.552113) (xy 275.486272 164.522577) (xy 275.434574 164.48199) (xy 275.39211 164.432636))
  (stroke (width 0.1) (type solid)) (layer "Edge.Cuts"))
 (gr_arc (start 283.321123 146.304) (mid 283.4979 146.377223) (end 283.571123 146.554) (stroke (width 0.1) (type solid)) (layer "Edge.Cuts"))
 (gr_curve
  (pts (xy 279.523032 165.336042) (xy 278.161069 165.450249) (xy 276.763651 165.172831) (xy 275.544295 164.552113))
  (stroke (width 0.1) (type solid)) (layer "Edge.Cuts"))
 (gr_arc (start 274.271123 146.554) (mid 274.344346 146.377223) (end 274.521123 146.304) (stroke (width 0.1) (type solid))
  (layer "Edge.Cuts"))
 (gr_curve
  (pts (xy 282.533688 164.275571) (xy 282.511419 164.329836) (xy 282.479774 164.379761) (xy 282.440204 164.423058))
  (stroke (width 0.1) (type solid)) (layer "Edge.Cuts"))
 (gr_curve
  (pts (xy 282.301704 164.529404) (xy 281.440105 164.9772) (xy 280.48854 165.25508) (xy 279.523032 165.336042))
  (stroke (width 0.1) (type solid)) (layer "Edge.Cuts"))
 (gr_line (start 279.7048 146.304) (end 274.521123 146.304) (stroke (width 0.1) (type solid)) (layer "Edge.Cuts"))
 (gr_arc (start 283.571123 149.554) (mid 283.4979 149.730777) (end 283.321123 149.804) (stroke (width 0.1) (type solid)) (layer "Edge.Cuts"))
 (segment (start 275.9964 158.366077) (end 275.9964 153.797) (width 0.25) (layer "F.Cu") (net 1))
 (segment (start 276.584323 158.954) (end 275.9964 158.366077) (width 0.25) (layer "F.Cu") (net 1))
 (segment (start 275.9964 153.797) (end 276.535963 153.257437) (width 0.25) (layer "F.Cu") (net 1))
 (segment (start 276.535963 153.257437) (end 276.535963 147.415545) (width 0.25) (layer "F.Cu") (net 1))
 (segment (start 279.135963 147.415545) (end 279.135963 152.872563) (width 0.25) (layer "F.Cu") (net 2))
 (segment (start 281.813 155.5496) (end 281.813 158.831485) (width 0.25) (layer "F.Cu") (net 2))
 (segment (start 279.135963 152.872563) (end 281.813 155.5496) (width 0.25) (layer "F.Cu") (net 2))
 (segment (start 281.813 158.831485) (end 281.690386 158.954099) (width 0.25) (layer "F.Cu") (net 2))
 (segment (start 281.690386 158.954099) (end 281.170778 158.954099) (width 0.25) (layer "F.Cu") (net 2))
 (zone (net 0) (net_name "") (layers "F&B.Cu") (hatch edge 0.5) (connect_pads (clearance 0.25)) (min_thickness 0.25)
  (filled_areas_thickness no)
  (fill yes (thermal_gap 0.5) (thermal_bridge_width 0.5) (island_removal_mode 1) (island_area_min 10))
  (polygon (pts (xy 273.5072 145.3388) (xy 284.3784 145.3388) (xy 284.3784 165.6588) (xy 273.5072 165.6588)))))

